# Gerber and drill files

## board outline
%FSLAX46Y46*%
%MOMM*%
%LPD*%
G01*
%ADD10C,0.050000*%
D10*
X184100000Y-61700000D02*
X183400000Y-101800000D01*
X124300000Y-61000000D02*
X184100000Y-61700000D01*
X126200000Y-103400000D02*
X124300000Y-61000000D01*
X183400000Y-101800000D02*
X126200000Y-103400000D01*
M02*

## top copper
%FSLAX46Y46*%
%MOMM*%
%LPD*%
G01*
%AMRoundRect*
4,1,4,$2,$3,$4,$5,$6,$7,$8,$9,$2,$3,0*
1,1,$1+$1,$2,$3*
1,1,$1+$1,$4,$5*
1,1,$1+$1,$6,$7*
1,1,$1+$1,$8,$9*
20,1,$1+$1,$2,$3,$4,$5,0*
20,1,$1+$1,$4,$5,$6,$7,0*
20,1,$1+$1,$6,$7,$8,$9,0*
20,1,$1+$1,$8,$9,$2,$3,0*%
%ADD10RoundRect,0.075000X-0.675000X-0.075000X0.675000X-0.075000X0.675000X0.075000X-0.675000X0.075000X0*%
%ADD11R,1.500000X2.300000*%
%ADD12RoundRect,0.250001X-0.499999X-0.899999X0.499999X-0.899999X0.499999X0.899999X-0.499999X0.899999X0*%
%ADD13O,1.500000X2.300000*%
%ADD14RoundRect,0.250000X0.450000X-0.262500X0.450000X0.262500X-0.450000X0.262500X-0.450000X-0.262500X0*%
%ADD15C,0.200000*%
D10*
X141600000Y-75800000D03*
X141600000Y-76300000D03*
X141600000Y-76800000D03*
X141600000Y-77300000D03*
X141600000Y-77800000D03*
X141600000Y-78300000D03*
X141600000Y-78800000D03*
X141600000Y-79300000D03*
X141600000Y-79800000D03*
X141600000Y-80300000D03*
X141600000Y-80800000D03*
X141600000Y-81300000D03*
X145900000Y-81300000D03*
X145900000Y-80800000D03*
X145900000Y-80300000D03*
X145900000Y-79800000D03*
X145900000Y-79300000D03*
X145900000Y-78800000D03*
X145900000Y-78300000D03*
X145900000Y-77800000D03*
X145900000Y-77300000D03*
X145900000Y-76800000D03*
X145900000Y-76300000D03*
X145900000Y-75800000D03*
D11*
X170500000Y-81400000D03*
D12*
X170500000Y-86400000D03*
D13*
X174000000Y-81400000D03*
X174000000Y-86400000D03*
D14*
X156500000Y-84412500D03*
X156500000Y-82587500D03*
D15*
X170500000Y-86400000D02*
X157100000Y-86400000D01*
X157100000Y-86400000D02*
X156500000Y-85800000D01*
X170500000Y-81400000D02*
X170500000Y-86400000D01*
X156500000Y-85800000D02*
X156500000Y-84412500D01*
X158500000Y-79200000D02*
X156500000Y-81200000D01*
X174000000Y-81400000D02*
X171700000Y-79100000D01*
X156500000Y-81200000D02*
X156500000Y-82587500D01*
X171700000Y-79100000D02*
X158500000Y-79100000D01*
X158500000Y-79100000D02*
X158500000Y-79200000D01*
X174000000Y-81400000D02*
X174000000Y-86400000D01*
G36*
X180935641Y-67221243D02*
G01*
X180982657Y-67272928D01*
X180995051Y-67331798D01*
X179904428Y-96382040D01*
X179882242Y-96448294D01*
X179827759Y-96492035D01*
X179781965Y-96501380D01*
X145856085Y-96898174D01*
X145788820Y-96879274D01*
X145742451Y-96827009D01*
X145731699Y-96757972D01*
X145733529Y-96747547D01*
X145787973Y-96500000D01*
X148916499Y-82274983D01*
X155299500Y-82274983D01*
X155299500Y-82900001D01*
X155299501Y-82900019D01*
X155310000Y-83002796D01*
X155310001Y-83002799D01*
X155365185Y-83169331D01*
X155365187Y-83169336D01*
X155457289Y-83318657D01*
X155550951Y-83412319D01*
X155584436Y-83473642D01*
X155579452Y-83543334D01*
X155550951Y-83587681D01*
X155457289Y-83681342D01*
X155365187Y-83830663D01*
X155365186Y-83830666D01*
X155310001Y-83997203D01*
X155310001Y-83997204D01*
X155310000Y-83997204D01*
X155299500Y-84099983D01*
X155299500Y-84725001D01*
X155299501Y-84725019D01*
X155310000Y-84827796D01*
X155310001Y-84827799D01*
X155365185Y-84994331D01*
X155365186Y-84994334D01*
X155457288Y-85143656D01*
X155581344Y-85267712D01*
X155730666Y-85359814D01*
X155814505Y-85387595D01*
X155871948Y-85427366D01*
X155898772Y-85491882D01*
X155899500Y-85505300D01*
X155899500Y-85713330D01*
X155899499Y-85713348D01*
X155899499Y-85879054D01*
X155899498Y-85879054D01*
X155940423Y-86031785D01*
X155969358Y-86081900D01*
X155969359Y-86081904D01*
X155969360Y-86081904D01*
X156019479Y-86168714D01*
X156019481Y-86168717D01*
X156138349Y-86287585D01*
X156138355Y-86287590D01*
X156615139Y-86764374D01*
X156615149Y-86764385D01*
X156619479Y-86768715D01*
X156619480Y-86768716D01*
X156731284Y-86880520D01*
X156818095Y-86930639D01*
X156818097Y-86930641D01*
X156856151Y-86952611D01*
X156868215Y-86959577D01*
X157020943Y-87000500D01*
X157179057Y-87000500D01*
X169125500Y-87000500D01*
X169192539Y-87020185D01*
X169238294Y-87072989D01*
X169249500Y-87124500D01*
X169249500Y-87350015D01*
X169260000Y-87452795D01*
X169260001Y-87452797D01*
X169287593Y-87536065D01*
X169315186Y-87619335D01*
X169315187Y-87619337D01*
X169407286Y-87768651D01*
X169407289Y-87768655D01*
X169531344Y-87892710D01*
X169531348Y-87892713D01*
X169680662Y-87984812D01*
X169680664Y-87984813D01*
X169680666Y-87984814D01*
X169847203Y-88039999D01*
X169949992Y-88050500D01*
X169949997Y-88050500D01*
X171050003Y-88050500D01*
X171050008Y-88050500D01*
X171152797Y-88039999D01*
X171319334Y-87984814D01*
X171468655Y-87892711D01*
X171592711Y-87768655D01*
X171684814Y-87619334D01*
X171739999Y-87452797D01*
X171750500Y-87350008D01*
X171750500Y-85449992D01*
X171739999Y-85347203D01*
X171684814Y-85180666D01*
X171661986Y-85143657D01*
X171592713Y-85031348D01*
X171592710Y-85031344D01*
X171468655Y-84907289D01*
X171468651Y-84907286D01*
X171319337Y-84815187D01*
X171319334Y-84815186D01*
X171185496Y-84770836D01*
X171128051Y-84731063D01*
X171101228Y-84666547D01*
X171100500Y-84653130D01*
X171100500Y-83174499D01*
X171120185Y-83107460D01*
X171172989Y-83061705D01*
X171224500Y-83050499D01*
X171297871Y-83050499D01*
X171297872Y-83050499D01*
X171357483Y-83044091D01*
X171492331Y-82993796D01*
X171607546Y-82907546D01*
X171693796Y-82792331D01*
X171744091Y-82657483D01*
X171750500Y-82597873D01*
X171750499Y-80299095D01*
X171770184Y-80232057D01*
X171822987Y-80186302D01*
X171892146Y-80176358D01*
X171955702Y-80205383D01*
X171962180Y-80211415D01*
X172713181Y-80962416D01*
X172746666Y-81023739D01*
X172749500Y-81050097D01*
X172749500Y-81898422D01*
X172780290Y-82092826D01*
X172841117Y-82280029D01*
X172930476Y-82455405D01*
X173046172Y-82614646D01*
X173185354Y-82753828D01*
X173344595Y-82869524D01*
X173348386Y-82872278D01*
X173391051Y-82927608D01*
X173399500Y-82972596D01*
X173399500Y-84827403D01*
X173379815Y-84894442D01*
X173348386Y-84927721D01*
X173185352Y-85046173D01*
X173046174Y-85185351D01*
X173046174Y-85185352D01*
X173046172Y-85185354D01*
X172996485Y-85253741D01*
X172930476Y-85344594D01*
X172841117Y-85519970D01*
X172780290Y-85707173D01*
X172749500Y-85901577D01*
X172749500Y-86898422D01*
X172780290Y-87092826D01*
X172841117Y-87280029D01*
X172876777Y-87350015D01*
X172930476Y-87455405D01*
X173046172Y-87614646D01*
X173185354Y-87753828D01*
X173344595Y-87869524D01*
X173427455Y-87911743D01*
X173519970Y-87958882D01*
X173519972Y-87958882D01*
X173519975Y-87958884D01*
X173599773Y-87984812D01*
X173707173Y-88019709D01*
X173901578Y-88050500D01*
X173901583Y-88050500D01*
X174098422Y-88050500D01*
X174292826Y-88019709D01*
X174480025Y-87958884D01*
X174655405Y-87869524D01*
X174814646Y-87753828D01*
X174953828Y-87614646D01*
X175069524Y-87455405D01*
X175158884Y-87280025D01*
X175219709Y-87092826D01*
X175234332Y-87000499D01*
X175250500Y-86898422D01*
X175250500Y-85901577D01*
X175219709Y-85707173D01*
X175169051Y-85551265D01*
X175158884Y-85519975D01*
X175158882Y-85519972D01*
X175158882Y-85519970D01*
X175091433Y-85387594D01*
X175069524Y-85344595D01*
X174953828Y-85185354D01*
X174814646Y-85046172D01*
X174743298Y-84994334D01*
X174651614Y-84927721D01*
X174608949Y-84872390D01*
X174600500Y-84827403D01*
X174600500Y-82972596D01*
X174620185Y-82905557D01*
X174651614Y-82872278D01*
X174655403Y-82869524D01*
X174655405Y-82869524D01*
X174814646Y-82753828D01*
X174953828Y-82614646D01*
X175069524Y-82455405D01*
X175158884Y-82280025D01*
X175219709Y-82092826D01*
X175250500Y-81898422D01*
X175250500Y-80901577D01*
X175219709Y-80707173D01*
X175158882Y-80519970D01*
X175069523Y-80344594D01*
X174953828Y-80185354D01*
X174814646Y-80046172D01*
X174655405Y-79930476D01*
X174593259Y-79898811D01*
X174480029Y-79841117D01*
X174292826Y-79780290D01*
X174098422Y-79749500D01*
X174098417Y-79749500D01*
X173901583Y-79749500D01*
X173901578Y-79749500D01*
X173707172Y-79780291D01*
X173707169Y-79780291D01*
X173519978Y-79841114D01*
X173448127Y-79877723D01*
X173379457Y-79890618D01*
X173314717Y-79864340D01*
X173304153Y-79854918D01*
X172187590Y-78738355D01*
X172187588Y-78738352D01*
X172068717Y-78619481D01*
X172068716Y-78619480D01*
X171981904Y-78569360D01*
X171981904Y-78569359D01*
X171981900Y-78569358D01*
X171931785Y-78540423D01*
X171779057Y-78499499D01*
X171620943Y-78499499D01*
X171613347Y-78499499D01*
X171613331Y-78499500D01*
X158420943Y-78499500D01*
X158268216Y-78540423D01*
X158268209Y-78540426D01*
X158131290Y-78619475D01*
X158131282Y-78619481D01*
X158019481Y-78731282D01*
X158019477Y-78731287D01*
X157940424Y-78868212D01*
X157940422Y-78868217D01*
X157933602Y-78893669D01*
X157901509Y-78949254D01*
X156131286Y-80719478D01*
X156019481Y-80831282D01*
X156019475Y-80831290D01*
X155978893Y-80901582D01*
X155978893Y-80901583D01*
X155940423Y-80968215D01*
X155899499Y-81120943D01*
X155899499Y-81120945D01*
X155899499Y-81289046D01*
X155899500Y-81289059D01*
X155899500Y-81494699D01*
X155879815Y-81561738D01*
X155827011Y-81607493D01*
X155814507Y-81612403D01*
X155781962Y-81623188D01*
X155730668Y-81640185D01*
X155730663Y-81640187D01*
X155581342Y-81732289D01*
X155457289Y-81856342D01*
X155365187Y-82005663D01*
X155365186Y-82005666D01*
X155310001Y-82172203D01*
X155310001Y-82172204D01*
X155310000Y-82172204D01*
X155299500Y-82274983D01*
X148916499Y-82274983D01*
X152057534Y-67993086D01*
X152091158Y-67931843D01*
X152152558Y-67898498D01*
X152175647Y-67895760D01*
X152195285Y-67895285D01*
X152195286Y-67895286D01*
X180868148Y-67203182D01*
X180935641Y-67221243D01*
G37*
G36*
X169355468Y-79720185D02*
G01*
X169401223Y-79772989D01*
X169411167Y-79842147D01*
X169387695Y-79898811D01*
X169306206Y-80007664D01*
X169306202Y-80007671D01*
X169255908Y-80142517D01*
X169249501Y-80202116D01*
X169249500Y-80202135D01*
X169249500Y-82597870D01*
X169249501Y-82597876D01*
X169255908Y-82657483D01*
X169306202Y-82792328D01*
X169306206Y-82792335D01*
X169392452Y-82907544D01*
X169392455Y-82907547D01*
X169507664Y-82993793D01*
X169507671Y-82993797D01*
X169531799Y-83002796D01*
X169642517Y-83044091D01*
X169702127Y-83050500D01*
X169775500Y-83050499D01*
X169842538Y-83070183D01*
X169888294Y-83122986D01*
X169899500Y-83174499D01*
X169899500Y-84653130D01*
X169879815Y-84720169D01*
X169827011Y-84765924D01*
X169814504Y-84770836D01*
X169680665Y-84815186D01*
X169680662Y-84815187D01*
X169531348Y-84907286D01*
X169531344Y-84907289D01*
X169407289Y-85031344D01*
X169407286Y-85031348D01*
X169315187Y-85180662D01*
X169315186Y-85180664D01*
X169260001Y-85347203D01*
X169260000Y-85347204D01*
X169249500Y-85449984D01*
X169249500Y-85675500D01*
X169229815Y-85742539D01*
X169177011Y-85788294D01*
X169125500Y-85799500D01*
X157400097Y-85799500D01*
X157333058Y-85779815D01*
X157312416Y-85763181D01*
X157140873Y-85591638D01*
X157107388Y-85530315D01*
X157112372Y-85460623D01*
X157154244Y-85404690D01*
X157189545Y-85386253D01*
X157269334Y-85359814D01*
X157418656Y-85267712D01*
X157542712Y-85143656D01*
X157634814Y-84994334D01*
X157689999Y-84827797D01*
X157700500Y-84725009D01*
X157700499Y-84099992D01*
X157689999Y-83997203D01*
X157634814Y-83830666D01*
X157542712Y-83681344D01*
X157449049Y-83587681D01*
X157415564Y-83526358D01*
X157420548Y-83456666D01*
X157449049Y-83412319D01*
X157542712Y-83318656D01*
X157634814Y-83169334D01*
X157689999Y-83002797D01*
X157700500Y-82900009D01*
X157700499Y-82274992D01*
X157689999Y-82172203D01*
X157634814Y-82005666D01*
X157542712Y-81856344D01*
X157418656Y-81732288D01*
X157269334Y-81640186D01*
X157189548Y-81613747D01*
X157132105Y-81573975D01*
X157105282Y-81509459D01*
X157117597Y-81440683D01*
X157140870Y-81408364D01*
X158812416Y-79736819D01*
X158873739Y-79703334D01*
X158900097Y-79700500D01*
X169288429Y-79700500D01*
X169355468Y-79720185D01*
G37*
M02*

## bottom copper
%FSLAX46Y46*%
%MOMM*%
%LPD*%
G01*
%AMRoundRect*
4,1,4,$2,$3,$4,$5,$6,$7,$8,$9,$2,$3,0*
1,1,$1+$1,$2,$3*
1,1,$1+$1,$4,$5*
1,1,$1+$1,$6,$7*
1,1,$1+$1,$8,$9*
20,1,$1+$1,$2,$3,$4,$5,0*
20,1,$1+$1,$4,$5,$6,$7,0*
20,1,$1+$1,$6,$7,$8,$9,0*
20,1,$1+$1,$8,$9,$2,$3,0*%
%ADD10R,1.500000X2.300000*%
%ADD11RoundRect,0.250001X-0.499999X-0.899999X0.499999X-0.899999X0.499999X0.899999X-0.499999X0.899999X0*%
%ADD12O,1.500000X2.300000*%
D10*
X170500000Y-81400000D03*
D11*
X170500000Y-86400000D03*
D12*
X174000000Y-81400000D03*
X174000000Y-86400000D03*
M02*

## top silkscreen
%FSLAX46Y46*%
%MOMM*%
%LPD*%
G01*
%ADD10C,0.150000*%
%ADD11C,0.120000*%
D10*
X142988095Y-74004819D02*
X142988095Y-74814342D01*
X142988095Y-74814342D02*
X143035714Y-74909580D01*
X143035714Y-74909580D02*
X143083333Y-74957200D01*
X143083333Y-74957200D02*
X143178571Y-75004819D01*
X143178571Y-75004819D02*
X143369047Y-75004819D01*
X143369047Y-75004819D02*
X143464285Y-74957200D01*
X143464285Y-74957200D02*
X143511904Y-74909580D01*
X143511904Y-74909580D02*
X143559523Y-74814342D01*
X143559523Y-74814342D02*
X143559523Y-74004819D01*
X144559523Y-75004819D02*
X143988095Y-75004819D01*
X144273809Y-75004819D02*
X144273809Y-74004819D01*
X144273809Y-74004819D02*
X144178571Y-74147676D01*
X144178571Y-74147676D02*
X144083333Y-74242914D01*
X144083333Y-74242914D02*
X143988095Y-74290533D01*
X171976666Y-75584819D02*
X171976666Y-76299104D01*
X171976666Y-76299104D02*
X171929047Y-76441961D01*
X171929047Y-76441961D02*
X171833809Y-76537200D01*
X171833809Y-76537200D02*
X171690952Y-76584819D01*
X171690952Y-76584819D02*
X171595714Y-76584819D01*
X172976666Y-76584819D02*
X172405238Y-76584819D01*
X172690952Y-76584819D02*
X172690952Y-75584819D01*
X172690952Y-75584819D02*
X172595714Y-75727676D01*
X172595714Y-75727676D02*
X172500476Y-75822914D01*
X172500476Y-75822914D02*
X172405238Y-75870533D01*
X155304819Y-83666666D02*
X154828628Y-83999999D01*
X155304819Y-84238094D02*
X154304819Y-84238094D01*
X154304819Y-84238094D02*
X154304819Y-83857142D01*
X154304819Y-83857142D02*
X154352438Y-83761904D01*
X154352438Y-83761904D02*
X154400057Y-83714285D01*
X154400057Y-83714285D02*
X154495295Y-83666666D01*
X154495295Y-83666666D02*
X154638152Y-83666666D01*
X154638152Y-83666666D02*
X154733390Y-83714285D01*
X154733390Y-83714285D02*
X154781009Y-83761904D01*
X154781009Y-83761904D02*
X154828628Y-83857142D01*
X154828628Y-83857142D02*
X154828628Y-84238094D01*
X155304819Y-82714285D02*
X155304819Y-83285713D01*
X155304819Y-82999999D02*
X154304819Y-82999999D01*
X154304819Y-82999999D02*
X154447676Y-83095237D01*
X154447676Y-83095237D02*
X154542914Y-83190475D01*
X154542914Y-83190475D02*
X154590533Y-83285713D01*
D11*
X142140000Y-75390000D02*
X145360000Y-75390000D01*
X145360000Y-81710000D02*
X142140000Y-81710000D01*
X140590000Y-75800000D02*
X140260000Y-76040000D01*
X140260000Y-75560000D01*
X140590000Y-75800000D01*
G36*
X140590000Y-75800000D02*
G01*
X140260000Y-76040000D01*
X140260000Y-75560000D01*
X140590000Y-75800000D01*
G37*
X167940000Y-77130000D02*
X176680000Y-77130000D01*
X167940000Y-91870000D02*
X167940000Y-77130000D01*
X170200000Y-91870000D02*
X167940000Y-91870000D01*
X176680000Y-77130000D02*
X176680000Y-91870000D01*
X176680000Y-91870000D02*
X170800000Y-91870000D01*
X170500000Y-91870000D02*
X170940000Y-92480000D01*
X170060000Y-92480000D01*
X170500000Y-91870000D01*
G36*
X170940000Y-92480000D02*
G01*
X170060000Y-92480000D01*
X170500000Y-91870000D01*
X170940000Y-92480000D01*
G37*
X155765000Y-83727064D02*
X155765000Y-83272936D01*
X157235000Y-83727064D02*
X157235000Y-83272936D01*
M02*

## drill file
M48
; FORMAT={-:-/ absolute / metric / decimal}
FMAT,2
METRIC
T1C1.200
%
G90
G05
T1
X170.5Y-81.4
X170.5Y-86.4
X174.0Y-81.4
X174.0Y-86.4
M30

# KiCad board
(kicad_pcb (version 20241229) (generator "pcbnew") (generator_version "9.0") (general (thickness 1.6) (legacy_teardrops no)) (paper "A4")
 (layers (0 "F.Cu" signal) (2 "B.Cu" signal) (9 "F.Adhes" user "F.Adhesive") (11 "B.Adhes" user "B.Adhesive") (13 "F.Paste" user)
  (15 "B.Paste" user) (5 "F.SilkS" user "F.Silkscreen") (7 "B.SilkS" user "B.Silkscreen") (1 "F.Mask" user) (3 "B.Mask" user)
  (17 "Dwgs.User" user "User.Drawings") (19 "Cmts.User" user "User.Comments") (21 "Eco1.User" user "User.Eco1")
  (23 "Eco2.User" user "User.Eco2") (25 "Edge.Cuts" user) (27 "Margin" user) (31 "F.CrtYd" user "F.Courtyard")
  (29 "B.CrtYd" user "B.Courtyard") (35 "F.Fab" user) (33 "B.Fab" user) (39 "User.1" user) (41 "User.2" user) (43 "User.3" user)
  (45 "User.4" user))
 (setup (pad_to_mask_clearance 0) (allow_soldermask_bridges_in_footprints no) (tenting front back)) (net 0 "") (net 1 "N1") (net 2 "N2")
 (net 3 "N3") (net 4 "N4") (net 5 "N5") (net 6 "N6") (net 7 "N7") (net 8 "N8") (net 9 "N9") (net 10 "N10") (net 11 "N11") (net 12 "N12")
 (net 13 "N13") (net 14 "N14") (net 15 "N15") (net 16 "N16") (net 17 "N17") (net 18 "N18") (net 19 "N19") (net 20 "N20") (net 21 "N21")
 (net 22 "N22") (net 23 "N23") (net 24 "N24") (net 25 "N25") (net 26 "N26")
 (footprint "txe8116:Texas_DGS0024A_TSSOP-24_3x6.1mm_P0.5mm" (layer "F.Cu") (at 143.75 78.55)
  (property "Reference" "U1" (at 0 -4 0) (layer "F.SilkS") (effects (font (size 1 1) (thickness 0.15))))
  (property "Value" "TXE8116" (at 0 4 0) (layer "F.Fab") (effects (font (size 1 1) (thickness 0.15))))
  (fp_line (start -1.61 -3.16) (end 1.61 -3.16) (stroke (width 0.12) (type solid)) (layer "F.SilkS"))
  (fp_line (start 1.61 3.16) (end -1.61 3.16) (stroke (width 0.12) (type solid)) (layer "F.SilkS"))
  (fp_poly (pts (xy -3.16 -2.75) (xy -3.49 -2.51) (xy -3.49 -2.99)) (stroke (width 0.12) (type solid)) (fill yes) (layer "F.SilkS"))
  (pad "1" smd roundrect (at -2.15 -2.75) (size 1.5 0.3) (layers "F.Cu" "F.Mask" "F.Paste") (roundrect_rratio 0.25) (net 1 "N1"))
  (pad "2" smd roundrect (at -2.15 -2.25) (size 1.5 0.3) (layers "F.Cu" "F.Mask" "F.Paste") (roundrect_rratio 0.25) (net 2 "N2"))
  (pad "3" smd roundrect (at -2.15 -1.75) (size 1.5 0.3) (layers "F.Cu" "F.Mask" "F.Paste") (roundrect_rratio 0.25) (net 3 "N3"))
  (pad "4" smd roundrect (at -2.15 -1.25) (size 1.5 0.3) (layers "F.Cu" "F.Mask" "F.Paste") (roundrect_rratio 0.25) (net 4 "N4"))
  (pad "5" smd roundrect (at -2.15 -0.75) (size 1.5 0.3) (layers "F.Cu" "F.Mask" "F.Paste") (roundrect_rratio 0.25) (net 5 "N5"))
  (pad "6" smd roundrect (at -2.15 -0.25) (size 1.5 0.3) (layers "F.Cu" "F.Mask" "F.Paste") (roundrect_rratio 0.25) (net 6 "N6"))
  (pad "7" smd roundrect (at -2.15 0.25) (size 1.5 0.3) (layers "F.Cu" "F.Mask" "F.Paste") (roundrect_rratio 0.25) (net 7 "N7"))
  (pad "8" smd roundrect (at -2.15 0.75) (size 1.5 0.3) (layers "F.Cu" "F.Mask" "F.Paste") (roundrect_rratio 0.25) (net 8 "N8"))
  (pad "9" smd roundrect (at -2.15 1.25) (size 1.5 0.3) (layers "F.Cu" "F.Mask" "F.Paste") (roundrect_rratio 0.25) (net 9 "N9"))
  (pad "10" smd roundrect (at -2.15 1.75) (size 1.5 0.3) (layers "F.Cu" "F.Mask" "F.Paste") (roundrect_rratio 0.25) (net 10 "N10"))
  (pad "11" smd roundrect (at -2.15 2.25) (size 1.5 0.3) (layers "F.Cu" "F.Mask" "F.Paste") (roundrect_rratio 0.25) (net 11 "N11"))
  (pad "12" smd roundrect (at -2.15 2.75) (size 1.5 0.3) (layers "F.Cu" "F.Mask" "F.Paste") (roundrect_rratio 0.25) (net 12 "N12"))
  (pad "13" smd roundrect (at 2.15 2.75) (size 1.5 0.3) (layers "F.Cu" "F.Mask" "F.Paste") (roundrect_rratio 0.25) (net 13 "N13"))
  (pad "14" smd roundrect (at 2.15 2.25) (size 1.5 0.3) (layers "F.Cu" "F.Mask" "F.Paste") (roundrect_rratio 0.25) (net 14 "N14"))
  (pad "15" smd roundrect (at 2.15 1.75) (size 1.5 0.3) (layers "F.Cu" "F.Mask" "F.Paste") (roundrect_rratio 0.25) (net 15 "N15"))
  (pad "16" smd roundrect (at 2.15 1.25) (size 1.5 0.3) (layers "F.Cu" "F.Mask" "F.Paste") (roundrect_rratio 0.25) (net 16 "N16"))
  (pad "17" smd roundrect (at 2.15 0.75) (size 1.5 0.3) (layers "F.Cu" "F.Mask" "F.Paste") (roundrect_rratio 0.25) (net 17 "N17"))
  (pad "18" smd roundrect (at 2.15 0.25) (size 1.5 0.3) (layers "F.Cu" "F.Mask" "F.Paste") (roundrect_rratio 0.25) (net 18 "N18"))
  (pad "19" smd roundrect (at 2.15 -0.25) (size 1.5 0.3) (layers "F.Cu" "F.Mask" "F.Paste") (roundrect_rratio 0.25) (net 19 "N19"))
  (pad "20" smd roundrect (at 2.15 -0.75) (size 1.5 0.3) (layers "F.Cu" "F.Mask" "F.Paste") (roundrect_rratio 0.25) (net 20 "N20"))
  (pad "21" smd roundrect (at 2.15 -1.25) (size 1.5 0.3) (layers "F.Cu" "F.Mask" "F.Paste") (roundrect_rratio 0.25) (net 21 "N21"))
  (pad "22" smd roundrect (at 2.15 -1.75) (size 1.5 0.3) (layers "F.Cu" "F.Mask" "F.Paste") (roundrect_rratio 0.25) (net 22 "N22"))
  (pad "23" smd roundrect (at 2.15 -2.25) (size 1.5 0.3) (layers "F.Cu" "F.Mask" "F.Paste") (roundrect_rratio 0.25) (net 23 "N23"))
  (pad "24" smd roundrect (at 2.15 -2.75) (size 1.5 0.3) (layers "F.Cu" "F.Mask" "F.Paste") (roundrect_rratio 0.25) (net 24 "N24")))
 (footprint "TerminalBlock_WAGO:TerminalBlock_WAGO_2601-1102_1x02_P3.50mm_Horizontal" (layer "F.Cu") (at 170.5 86.4)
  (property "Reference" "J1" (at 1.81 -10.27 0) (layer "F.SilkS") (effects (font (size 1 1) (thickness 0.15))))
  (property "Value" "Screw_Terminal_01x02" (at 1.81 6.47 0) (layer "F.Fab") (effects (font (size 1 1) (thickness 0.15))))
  (fp_line (start -2.56 -9.27) (end 6.18 -9.27) (stroke (width 0.12) (type solid)) (layer "F.SilkS"))
  (fp_line (start -2.56 5.47) (end -2.56 -9.27) (stroke (width 0.12) (type solid)) (layer "F.SilkS"))
  (fp_line (start -0.3 5.47) (end -2.56 5.47) (stroke (width 0.12) (type solid)) (layer "F.SilkS"))
  (fp_line (start 6.18 -9.27) (end 6.18 5.47) (stroke (width 0.12) (type solid)) (layer "F.SilkS"))
  (fp_line (start 6.18 5.47) (end 0.3 5.47) (stroke (width 0.12) (type solid)) (layer "F.SilkS"))
  (fp_poly (pts (xy 0 5.47) (xy 0.44 6.08) (xy -0.44 6.08)) (stroke (width 0.12) (type solid)) (fill yes) (layer "F.SilkS"))
  (pad "1" thru_hole rect (at 0 -5) (size 1.5 2.3) (drill 1.2) (layers "*.Cu" "*.Mask") (remove_unused_layers no) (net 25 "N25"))
  (pad "1" thru_hole roundrect (at 0 0) (size 1.5 2.3) (drill 1.2) (layers "*.Cu" "*.Mask") (remove_unused_layers no)
   (roundrect_rratio 0.166667) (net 25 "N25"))
  (pad "2" thru_hole oval (at 3.5 -5) (size 1.5 2.3) (drill 1.2) (layers "*.Cu" "*.Mask") (remove_unused_layers no) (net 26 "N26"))
  (pad "2" thru_hole oval (at 3.5 0) (size 1.5 2.3) (drill 1.2) (layers "*.Cu" "*.Mask") (remove_unused_layers no) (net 26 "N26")))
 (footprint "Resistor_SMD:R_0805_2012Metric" (layer "F.Cu") (at 156.5 83.5 90)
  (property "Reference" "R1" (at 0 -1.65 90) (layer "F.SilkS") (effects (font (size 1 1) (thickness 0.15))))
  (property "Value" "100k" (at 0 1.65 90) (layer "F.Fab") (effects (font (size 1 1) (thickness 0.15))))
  (fp_line (start -0.227064 -0.735) (end 0.227064 -0.735) (stroke (width 0.12) (type solid)) (layer "F.SilkS"))
  (fp_line (start -0.227064 0.735) (end 0.227064 0.735) (stroke (width 0.12) (type solid)) (layer "F.SilkS"))
  (pad "1" smd roundrect (at -0.9125 0 90) (size 1.025 1.4) (layers "F.Cu" "F.Mask" "F.Paste") (roundrect_rratio 0.243902) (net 25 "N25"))
  (pad "2" smd roundrect (at 0.9125 0 90) (size 1.025 1.4) (layers "F.Cu" "F.Mask" "F.Paste") (roundrect_rratio 0.243902) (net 26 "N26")))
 (gr_line (start 184.1 61.7) (end 183.4 101.8) (stroke (width 0.05) (type default)) (layer "Edge.Cuts"))
 (gr_line (start 124.3 61) (end 184.1 61.7) (stroke (width 0.05) (type default)) (layer "Edge.Cuts"))
 (gr_line (start 126.2 103.4) (end 124.3 61) (stroke (width 0.05) (type default)) (layer "Edge.Cuts"))
 (gr_line (start 183.4 101.8) (end 126.2 103.4) (stroke (width 0.05) (type default)) (layer "Edge.Cuts"))
 (segment (start 170.5 86.4) (end 157.1 86.4) (width 0.2) (layer "F.Cu") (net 25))
 (segment (start 157.1 86.4) (end 156.5 85.8) (width 0.2) (layer "F.Cu") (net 25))
 (segment (start 170.5 81.4) (end 170.5 86.4) (width 0.2) (layer "F.Cu") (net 25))
 (segment (start 156.5 85.8) (end 156.5 84.4125) (width 0.2) (layer "F.Cu") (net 25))
 (segment (start 158.5 79.2) (end 156.5 81.2) (width 0.2) (layer "F.Cu") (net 26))
 (segment (start 174 81.4) (end 171.7 79.1) (width 0.2) (layer "F.Cu") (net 26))
 (segment (start 156.5 81.2) (end 156.5 82.5875) (width 0.2) (layer "F.Cu") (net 26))
 (segment (start 171.7 79.1) (end 158.5 79.1) (width 0.2) (layer "F.Cu") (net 26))
 (segment (start 158.5 79.1) (end 158.5 79.2) (width 0.2) (layer "F.Cu") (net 26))
 (segment (start 174 81.4) (end 174 86.4) (width 0.2) (layer "F.Cu") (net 26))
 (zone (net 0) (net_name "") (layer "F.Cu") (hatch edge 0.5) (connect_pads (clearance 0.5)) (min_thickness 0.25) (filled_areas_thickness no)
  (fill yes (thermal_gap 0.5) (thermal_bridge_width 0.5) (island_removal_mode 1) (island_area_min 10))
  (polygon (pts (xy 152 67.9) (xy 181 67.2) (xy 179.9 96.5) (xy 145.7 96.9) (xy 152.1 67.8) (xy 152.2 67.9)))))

